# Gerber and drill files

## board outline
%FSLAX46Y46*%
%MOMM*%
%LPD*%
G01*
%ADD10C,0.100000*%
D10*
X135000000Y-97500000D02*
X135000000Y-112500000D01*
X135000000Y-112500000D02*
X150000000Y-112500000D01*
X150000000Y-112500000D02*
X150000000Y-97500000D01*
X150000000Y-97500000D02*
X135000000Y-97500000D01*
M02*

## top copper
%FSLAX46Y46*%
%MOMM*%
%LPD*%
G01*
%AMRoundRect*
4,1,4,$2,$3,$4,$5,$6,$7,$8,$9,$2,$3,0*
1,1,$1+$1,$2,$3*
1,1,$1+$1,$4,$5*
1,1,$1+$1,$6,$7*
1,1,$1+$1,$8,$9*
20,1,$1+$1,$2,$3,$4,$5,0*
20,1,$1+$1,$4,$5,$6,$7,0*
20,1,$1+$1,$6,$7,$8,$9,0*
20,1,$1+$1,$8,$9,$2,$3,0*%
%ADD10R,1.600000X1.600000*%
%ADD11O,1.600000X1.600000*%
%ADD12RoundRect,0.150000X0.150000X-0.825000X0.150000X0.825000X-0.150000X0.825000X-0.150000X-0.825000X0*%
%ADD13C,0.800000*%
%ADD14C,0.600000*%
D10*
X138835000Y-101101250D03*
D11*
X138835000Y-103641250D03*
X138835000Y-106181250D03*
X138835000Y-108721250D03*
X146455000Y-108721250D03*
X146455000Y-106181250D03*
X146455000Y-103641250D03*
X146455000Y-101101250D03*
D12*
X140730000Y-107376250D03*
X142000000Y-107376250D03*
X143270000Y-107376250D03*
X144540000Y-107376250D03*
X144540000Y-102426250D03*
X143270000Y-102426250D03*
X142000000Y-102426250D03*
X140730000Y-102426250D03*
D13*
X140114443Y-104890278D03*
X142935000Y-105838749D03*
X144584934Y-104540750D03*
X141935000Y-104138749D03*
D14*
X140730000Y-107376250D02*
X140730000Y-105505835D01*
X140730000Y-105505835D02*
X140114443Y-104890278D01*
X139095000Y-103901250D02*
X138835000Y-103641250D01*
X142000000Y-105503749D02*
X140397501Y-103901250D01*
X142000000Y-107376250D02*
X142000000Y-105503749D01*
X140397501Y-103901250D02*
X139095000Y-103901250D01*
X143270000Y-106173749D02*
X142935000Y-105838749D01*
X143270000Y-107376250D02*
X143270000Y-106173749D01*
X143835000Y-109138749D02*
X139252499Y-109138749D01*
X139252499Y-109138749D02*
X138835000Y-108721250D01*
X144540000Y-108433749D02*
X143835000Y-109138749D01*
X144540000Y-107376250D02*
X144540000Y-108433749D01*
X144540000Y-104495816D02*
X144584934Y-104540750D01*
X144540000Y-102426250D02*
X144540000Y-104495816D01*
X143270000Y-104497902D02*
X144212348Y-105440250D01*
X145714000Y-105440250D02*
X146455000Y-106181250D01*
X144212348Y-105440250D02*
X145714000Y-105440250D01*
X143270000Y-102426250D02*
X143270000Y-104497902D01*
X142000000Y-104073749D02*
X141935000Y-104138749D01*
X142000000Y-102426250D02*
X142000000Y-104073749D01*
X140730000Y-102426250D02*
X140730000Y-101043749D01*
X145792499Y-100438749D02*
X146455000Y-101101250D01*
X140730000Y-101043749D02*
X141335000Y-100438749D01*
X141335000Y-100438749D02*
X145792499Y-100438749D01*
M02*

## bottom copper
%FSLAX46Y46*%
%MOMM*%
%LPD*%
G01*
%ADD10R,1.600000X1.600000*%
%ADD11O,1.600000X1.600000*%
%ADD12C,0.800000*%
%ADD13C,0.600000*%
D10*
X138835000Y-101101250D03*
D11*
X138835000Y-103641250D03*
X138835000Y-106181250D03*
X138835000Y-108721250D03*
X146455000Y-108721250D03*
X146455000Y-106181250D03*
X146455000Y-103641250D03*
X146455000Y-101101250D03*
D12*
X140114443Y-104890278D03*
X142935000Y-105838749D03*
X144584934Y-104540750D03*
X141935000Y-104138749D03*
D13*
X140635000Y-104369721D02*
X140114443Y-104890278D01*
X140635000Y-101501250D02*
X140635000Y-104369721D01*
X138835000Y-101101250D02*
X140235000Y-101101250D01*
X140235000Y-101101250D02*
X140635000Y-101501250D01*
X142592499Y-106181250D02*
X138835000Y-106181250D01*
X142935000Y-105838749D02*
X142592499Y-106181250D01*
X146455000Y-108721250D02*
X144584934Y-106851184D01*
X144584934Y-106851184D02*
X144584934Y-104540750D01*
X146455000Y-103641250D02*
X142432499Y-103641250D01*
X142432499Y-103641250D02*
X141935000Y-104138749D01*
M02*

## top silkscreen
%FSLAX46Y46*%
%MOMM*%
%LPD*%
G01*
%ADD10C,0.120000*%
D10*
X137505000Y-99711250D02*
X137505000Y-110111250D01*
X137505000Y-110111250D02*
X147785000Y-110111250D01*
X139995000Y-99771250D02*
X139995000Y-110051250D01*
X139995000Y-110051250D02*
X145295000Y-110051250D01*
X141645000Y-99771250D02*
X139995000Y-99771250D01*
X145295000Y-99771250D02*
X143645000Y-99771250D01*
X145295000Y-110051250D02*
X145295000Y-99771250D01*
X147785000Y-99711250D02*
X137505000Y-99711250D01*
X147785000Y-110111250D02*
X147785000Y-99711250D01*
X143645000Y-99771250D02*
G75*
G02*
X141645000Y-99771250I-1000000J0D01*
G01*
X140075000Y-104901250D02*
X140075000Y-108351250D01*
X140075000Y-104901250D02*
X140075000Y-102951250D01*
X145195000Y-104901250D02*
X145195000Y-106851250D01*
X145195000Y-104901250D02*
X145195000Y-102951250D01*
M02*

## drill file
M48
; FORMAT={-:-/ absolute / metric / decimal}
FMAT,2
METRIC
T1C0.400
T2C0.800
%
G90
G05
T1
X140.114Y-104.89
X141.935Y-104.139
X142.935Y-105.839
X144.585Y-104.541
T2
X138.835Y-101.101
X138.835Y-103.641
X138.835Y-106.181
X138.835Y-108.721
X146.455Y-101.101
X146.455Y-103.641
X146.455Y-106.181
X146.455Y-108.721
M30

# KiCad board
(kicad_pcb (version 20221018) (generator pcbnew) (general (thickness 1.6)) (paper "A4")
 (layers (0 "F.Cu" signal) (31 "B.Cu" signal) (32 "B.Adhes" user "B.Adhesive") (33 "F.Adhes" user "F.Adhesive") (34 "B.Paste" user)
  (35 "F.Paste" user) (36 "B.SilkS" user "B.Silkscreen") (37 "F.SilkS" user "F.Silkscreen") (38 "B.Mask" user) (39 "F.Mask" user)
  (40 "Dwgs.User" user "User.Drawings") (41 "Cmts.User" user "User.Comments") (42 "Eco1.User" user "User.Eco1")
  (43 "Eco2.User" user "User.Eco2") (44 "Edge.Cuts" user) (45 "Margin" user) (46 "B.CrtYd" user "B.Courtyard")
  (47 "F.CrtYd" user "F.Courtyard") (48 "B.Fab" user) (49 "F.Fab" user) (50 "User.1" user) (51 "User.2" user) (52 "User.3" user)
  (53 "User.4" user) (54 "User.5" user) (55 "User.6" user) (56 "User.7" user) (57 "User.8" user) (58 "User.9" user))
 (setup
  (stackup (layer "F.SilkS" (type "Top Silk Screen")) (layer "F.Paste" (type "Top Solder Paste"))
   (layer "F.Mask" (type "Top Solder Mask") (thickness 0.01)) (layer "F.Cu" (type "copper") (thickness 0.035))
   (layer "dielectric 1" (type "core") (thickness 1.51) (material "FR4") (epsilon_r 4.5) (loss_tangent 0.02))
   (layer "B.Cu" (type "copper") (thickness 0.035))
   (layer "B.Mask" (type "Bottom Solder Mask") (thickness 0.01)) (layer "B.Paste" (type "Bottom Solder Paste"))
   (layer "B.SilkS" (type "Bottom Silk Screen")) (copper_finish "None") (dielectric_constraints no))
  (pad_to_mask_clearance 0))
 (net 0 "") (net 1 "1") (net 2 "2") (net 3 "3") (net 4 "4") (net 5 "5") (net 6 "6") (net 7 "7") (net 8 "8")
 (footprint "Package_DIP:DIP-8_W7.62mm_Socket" (layer "F.Cu") (at 138.835 101.10125)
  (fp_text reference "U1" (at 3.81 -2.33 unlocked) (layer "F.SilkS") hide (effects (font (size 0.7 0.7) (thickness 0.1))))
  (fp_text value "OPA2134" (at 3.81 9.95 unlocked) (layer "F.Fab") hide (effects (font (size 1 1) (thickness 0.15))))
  (fp_line (start -1.33 -1.39) (end -1.33 9.01) (stroke (width 0.12) (type solid)) (layer "F.SilkS"))
  (fp_line (start -1.33 9.01) (end 8.95 9.01) (stroke (width 0.12) (type solid)) (layer "F.SilkS"))
  (fp_line (start 1.16 -1.33) (end 1.16 8.95) (stroke (width 0.12) (type solid)) (layer "F.SilkS"))
  (fp_line (start 1.16 8.95) (end 6.46 8.95) (stroke (width 0.12) (type solid)) (layer "F.SilkS"))
  (fp_line (start 2.81 -1.33) (end 1.16 -1.33) (stroke (width 0.12) (type solid)) (layer "F.SilkS"))
  (fp_line (start 6.46 -1.33) (end 4.81 -1.33) (stroke (width 0.12) (type solid)) (layer "F.SilkS"))
  (fp_line (start 6.46 8.95) (end 6.46 -1.33) (stroke (width 0.12) (type solid)) (layer "F.SilkS"))
  (fp_line (start 8.95 -1.39) (end -1.33 -1.39) (stroke (width 0.12) (type solid)) (layer "F.SilkS"))
  (fp_line (start 8.95 9.01) (end 8.95 -1.39) (stroke (width 0.12) (type solid)) (layer "F.SilkS"))
  (fp_arc (start 4.81 -1.33) (mid 3.81 -0.33) (end 2.81 -1.33) (stroke (width 0.12) (type solid)) (layer "F.SilkS"))
  (pad "1" thru_hole rect (at 0 0) (size 1.6 1.6) (drill 0.8) (layers "*.Cu" "*.Mask") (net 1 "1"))
  (pad "2" thru_hole oval (at 0 2.54) (size 1.6 1.6) (drill 0.8) (layers "*.Cu" "*.Mask") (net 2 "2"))
  (pad "3" thru_hole oval (at 0 5.08) (size 1.6 1.6) (drill 0.8) (layers "*.Cu" "*.Mask") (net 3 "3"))
  (pad "4" thru_hole oval (at 0 7.62) (size 1.6 1.6) (drill 0.8) (layers "*.Cu" "*.Mask") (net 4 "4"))
  (pad "5" thru_hole oval (at 7.62 7.62) (size 1.6 1.6) (drill 0.8) (layers "*.Cu" "*.Mask") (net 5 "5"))
  (pad "6" thru_hole oval (at 7.62 5.08) (size 1.6 1.6) (drill 0.8) (layers "*.Cu" "*.Mask") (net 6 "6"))
  (pad "7" thru_hole oval (at 7.62 2.54) (size 1.6 1.6) (drill 0.8) (layers "*.Cu" "*.Mask") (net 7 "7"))
  (pad "8" thru_hole oval (at 7.62 0) (size 1.6 1.6) (drill 0.8) (layers "*.Cu" "*.Mask") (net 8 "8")))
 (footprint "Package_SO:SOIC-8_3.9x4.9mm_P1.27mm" (layer "F.Cu") (at 142.635 104.90125 90)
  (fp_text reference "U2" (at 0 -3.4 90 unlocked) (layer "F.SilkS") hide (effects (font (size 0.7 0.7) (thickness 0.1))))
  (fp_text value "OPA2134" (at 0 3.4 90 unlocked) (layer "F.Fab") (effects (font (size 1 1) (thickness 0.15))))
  (fp_line (start 0 -2.56) (end -3.45 -2.56) (stroke (width 0.12) (type solid)) (layer "F.SilkS"))
  (fp_line (start 0 -2.56) (end 1.95 -2.56) (stroke (width 0.12) (type solid)) (layer "F.SilkS"))
  (fp_line (start 0 2.56) (end -1.95 2.56) (stroke (width 0.12) (type solid)) (layer "F.SilkS"))
  (fp_line (start 0 2.56) (end 1.95 2.56) (stroke (width 0.12) (type solid)) (layer "F.SilkS"))
  (pad "1" smd roundrect (at -2.475 -1.905 90) (size 1.95 0.6) (layers "F.Cu" "F.Paste" "F.Mask") (roundrect_rratio 0.25) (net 1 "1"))
  (pad "2" smd roundrect (at -2.475 -0.635 90) (size 1.95 0.6) (layers "F.Cu" "F.Paste" "F.Mask") (roundrect_rratio 0.25) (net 2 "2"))
  (pad "3" smd roundrect (at -2.475 0.635 90) (size 1.95 0.6) (layers "F.Cu" "F.Paste" "F.Mask") (roundrect_rratio 0.25) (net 3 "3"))
  (pad "4" smd roundrect (at -2.475 1.905 90) (size 1.95 0.6) (layers "F.Cu" "F.Paste" "F.Mask") (roundrect_rratio 0.25) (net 4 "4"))
  (pad "5" smd roundrect (at 2.475 1.905 90) (size 1.95 0.6) (layers "F.Cu" "F.Paste" "F.Mask") (roundrect_rratio 0.25) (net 5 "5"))
  (pad "6" smd roundrect (at 2.475 0.635 90) (size 1.95 0.6) (layers "F.Cu" "F.Paste" "F.Mask") (roundrect_rratio 0.25) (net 6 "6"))
  (pad "7" smd roundrect (at 2.475 -0.635 90) (size 1.95 0.6) (layers "F.Cu" "F.Paste" "F.Mask") (roundrect_rratio 0.25) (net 7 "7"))
  (pad "8" smd roundrect (at 2.475 -1.905 90) (size 1.95 0.6) (layers "F.Cu" "F.Paste" "F.Mask") (roundrect_rratio 0.25) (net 8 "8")))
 (gr_line (start 135 97.5) (end 135 112.5) (stroke (width 0.1) (type default)) (layer "Edge.Cuts"))
 (gr_line (start 135 112.5) (end 150 112.5) (stroke (width 0.1) (type default)) (layer "Edge.Cuts"))
 (gr_line (start 150 112.5) (end 150 97.5) (stroke (width 0.1) (type default)) (layer "Edge.Cuts"))
 (gr_line (start 150 97.5) (end 135 97.5) (stroke (width 0.1) (type default)) (layer "Edge.Cuts"))
 (segment (start 140.73 107.37625) (end 140.73 105.505835) (width 0.6) (layer "F.Cu") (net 1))
 (segment (start 140.73 105.505835) (end 140.114443 104.890278) (width 0.6) (layer "F.Cu") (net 1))
 (via (at 140.114443 104.890278) (size 0.8) (drill 0.4) (layers "F.Cu" "B.Cu") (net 1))
 (segment (start 140.635 104.369721) (end 140.114443 104.890278) (width 0.6) (layer "B.Cu") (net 1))
 (segment (start 140.635 101.50125) (end 140.635 104.369721) (width 0.6) (layer "B.Cu") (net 1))
 (segment (start 138.835 101.10125) (end 140.235 101.10125) (width 0.6) (layer "B.Cu") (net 1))
 (segment (start 140.235 101.10125) (end 140.635 101.50125) (width 0.6) (layer "B.Cu") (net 1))
 (segment (start 139.095 103.90125) (end 138.835 103.64125) (width 0.6) (layer "F.Cu") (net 2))
 (segment (start 142 105.503749) (end 140.397501 103.90125) (width 0.6) (layer "F.Cu") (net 2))
 (segment (start 142 107.37625) (end 142 105.503749) (width 0.6) (layer "F.Cu") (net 2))
 (segment (start 140.397501 103.90125) (end 139.095 103.90125) (width 0.6) (layer "F.Cu") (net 2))
 (segment (start 143.27 106.173749) (end 142.935 105.838749) (width 0.6) (layer "F.Cu") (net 3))
 (segment (start 143.27 107.37625) (end 143.27 106.173749) (width 0.6) (layer "F.Cu") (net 3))
 (via (at 142.935 105.838749) (size 0.8) (drill 0.4) (layers "F.Cu" "B.Cu") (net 3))
 (segment (start 142.592499 106.18125) (end 138.835 106.18125) (width 0.6) (layer "B.Cu") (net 3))
 (segment (start 142.935 105.838749) (end 142.592499 106.18125) (width 0.6) (layer "B.Cu") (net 3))
 (segment (start 143.835 109.138749) (end 139.252499 109.138749) (width 0.6) (layer "F.Cu") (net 4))
 (segment (start 139.252499 109.138749) (end 138.835 108.72125) (width 0.6) (layer "F.Cu") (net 4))
 (segment (start 144.54 108.433749) (end 143.835 109.138749) (width 0.6) (layer "F.Cu") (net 4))
 (segment (start 144.54 107.37625) (end 144.54 108.433749) (width 0.6) (layer "F.Cu") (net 4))
 (segment (start 144.54 104.495816) (end 144.584934 104.54075) (width 0.6) (layer "F.Cu") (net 5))
 (segment (start 144.54 102.42625) (end 144.54 104.495816) (width 0.6) (layer "F.Cu") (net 5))
 (via (at 144.584934 104.54075) (size 0.8) (drill 0.4) (layers "F.Cu" "B.Cu") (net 5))
 (segment (start 146.455 108.72125) (end 144.584934 106.851184) (width 0.6) (layer "B.Cu") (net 5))
 (segment (start 144.584934 106.851184) (end 144.584934 104.54075) (width 0.6) (layer "B.Cu") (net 5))
 (segment (start 143.27 104.497902) (end 144.212348 105.44025) (width 0.6) (layer "F.Cu") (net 6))
 (segment (start 145.714 105.44025) (end 146.455 106.18125) (width 0.6) (layer "F.Cu") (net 6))
 (segment (start 144.212348 105.44025) (end 145.714 105.44025) (width 0.6) (layer "F.Cu") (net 6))
 (segment (start 143.27 102.42625) (end 143.27 104.497902) (width 0.6) (layer "F.Cu") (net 6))
 (segment (start 142 104.073749) (end 141.935 104.138749) (width 0.6) (layer "F.Cu") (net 7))
 (segment (start 142 102.42625) (end 142 104.073749) (width 0.6) (layer "F.Cu") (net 7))
 (via (at 141.935 104.138749) (size 0.8) (drill 0.4) (layers "F.Cu" "B.Cu") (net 7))
 (segment (start 146.455 103.64125) (end 142.432499 103.64125) (width 0.6) (layer "B.Cu") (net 7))
 (segment (start 142.432499 103.64125) (end 141.935 104.138749) (width 0.6) (layer "B.Cu") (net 7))
 (segment (start 140.73 102.42625) (end 140.73 101.043749) (width 0.6) (layer "F.Cu") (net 8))
 (segment (start 145.792499 100.438749) (end 146.455 101.10125) (width 0.6) (layer "F.Cu") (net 8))
 (segment (start 140.73 101.043749) (end 141.335 100.438749) (width 0.6) (layer "F.Cu") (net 8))
 (segment (start 141.335 100.438749) (end 145.792499 100.438749) (width 0.6) (layer "F.Cu") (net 8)))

